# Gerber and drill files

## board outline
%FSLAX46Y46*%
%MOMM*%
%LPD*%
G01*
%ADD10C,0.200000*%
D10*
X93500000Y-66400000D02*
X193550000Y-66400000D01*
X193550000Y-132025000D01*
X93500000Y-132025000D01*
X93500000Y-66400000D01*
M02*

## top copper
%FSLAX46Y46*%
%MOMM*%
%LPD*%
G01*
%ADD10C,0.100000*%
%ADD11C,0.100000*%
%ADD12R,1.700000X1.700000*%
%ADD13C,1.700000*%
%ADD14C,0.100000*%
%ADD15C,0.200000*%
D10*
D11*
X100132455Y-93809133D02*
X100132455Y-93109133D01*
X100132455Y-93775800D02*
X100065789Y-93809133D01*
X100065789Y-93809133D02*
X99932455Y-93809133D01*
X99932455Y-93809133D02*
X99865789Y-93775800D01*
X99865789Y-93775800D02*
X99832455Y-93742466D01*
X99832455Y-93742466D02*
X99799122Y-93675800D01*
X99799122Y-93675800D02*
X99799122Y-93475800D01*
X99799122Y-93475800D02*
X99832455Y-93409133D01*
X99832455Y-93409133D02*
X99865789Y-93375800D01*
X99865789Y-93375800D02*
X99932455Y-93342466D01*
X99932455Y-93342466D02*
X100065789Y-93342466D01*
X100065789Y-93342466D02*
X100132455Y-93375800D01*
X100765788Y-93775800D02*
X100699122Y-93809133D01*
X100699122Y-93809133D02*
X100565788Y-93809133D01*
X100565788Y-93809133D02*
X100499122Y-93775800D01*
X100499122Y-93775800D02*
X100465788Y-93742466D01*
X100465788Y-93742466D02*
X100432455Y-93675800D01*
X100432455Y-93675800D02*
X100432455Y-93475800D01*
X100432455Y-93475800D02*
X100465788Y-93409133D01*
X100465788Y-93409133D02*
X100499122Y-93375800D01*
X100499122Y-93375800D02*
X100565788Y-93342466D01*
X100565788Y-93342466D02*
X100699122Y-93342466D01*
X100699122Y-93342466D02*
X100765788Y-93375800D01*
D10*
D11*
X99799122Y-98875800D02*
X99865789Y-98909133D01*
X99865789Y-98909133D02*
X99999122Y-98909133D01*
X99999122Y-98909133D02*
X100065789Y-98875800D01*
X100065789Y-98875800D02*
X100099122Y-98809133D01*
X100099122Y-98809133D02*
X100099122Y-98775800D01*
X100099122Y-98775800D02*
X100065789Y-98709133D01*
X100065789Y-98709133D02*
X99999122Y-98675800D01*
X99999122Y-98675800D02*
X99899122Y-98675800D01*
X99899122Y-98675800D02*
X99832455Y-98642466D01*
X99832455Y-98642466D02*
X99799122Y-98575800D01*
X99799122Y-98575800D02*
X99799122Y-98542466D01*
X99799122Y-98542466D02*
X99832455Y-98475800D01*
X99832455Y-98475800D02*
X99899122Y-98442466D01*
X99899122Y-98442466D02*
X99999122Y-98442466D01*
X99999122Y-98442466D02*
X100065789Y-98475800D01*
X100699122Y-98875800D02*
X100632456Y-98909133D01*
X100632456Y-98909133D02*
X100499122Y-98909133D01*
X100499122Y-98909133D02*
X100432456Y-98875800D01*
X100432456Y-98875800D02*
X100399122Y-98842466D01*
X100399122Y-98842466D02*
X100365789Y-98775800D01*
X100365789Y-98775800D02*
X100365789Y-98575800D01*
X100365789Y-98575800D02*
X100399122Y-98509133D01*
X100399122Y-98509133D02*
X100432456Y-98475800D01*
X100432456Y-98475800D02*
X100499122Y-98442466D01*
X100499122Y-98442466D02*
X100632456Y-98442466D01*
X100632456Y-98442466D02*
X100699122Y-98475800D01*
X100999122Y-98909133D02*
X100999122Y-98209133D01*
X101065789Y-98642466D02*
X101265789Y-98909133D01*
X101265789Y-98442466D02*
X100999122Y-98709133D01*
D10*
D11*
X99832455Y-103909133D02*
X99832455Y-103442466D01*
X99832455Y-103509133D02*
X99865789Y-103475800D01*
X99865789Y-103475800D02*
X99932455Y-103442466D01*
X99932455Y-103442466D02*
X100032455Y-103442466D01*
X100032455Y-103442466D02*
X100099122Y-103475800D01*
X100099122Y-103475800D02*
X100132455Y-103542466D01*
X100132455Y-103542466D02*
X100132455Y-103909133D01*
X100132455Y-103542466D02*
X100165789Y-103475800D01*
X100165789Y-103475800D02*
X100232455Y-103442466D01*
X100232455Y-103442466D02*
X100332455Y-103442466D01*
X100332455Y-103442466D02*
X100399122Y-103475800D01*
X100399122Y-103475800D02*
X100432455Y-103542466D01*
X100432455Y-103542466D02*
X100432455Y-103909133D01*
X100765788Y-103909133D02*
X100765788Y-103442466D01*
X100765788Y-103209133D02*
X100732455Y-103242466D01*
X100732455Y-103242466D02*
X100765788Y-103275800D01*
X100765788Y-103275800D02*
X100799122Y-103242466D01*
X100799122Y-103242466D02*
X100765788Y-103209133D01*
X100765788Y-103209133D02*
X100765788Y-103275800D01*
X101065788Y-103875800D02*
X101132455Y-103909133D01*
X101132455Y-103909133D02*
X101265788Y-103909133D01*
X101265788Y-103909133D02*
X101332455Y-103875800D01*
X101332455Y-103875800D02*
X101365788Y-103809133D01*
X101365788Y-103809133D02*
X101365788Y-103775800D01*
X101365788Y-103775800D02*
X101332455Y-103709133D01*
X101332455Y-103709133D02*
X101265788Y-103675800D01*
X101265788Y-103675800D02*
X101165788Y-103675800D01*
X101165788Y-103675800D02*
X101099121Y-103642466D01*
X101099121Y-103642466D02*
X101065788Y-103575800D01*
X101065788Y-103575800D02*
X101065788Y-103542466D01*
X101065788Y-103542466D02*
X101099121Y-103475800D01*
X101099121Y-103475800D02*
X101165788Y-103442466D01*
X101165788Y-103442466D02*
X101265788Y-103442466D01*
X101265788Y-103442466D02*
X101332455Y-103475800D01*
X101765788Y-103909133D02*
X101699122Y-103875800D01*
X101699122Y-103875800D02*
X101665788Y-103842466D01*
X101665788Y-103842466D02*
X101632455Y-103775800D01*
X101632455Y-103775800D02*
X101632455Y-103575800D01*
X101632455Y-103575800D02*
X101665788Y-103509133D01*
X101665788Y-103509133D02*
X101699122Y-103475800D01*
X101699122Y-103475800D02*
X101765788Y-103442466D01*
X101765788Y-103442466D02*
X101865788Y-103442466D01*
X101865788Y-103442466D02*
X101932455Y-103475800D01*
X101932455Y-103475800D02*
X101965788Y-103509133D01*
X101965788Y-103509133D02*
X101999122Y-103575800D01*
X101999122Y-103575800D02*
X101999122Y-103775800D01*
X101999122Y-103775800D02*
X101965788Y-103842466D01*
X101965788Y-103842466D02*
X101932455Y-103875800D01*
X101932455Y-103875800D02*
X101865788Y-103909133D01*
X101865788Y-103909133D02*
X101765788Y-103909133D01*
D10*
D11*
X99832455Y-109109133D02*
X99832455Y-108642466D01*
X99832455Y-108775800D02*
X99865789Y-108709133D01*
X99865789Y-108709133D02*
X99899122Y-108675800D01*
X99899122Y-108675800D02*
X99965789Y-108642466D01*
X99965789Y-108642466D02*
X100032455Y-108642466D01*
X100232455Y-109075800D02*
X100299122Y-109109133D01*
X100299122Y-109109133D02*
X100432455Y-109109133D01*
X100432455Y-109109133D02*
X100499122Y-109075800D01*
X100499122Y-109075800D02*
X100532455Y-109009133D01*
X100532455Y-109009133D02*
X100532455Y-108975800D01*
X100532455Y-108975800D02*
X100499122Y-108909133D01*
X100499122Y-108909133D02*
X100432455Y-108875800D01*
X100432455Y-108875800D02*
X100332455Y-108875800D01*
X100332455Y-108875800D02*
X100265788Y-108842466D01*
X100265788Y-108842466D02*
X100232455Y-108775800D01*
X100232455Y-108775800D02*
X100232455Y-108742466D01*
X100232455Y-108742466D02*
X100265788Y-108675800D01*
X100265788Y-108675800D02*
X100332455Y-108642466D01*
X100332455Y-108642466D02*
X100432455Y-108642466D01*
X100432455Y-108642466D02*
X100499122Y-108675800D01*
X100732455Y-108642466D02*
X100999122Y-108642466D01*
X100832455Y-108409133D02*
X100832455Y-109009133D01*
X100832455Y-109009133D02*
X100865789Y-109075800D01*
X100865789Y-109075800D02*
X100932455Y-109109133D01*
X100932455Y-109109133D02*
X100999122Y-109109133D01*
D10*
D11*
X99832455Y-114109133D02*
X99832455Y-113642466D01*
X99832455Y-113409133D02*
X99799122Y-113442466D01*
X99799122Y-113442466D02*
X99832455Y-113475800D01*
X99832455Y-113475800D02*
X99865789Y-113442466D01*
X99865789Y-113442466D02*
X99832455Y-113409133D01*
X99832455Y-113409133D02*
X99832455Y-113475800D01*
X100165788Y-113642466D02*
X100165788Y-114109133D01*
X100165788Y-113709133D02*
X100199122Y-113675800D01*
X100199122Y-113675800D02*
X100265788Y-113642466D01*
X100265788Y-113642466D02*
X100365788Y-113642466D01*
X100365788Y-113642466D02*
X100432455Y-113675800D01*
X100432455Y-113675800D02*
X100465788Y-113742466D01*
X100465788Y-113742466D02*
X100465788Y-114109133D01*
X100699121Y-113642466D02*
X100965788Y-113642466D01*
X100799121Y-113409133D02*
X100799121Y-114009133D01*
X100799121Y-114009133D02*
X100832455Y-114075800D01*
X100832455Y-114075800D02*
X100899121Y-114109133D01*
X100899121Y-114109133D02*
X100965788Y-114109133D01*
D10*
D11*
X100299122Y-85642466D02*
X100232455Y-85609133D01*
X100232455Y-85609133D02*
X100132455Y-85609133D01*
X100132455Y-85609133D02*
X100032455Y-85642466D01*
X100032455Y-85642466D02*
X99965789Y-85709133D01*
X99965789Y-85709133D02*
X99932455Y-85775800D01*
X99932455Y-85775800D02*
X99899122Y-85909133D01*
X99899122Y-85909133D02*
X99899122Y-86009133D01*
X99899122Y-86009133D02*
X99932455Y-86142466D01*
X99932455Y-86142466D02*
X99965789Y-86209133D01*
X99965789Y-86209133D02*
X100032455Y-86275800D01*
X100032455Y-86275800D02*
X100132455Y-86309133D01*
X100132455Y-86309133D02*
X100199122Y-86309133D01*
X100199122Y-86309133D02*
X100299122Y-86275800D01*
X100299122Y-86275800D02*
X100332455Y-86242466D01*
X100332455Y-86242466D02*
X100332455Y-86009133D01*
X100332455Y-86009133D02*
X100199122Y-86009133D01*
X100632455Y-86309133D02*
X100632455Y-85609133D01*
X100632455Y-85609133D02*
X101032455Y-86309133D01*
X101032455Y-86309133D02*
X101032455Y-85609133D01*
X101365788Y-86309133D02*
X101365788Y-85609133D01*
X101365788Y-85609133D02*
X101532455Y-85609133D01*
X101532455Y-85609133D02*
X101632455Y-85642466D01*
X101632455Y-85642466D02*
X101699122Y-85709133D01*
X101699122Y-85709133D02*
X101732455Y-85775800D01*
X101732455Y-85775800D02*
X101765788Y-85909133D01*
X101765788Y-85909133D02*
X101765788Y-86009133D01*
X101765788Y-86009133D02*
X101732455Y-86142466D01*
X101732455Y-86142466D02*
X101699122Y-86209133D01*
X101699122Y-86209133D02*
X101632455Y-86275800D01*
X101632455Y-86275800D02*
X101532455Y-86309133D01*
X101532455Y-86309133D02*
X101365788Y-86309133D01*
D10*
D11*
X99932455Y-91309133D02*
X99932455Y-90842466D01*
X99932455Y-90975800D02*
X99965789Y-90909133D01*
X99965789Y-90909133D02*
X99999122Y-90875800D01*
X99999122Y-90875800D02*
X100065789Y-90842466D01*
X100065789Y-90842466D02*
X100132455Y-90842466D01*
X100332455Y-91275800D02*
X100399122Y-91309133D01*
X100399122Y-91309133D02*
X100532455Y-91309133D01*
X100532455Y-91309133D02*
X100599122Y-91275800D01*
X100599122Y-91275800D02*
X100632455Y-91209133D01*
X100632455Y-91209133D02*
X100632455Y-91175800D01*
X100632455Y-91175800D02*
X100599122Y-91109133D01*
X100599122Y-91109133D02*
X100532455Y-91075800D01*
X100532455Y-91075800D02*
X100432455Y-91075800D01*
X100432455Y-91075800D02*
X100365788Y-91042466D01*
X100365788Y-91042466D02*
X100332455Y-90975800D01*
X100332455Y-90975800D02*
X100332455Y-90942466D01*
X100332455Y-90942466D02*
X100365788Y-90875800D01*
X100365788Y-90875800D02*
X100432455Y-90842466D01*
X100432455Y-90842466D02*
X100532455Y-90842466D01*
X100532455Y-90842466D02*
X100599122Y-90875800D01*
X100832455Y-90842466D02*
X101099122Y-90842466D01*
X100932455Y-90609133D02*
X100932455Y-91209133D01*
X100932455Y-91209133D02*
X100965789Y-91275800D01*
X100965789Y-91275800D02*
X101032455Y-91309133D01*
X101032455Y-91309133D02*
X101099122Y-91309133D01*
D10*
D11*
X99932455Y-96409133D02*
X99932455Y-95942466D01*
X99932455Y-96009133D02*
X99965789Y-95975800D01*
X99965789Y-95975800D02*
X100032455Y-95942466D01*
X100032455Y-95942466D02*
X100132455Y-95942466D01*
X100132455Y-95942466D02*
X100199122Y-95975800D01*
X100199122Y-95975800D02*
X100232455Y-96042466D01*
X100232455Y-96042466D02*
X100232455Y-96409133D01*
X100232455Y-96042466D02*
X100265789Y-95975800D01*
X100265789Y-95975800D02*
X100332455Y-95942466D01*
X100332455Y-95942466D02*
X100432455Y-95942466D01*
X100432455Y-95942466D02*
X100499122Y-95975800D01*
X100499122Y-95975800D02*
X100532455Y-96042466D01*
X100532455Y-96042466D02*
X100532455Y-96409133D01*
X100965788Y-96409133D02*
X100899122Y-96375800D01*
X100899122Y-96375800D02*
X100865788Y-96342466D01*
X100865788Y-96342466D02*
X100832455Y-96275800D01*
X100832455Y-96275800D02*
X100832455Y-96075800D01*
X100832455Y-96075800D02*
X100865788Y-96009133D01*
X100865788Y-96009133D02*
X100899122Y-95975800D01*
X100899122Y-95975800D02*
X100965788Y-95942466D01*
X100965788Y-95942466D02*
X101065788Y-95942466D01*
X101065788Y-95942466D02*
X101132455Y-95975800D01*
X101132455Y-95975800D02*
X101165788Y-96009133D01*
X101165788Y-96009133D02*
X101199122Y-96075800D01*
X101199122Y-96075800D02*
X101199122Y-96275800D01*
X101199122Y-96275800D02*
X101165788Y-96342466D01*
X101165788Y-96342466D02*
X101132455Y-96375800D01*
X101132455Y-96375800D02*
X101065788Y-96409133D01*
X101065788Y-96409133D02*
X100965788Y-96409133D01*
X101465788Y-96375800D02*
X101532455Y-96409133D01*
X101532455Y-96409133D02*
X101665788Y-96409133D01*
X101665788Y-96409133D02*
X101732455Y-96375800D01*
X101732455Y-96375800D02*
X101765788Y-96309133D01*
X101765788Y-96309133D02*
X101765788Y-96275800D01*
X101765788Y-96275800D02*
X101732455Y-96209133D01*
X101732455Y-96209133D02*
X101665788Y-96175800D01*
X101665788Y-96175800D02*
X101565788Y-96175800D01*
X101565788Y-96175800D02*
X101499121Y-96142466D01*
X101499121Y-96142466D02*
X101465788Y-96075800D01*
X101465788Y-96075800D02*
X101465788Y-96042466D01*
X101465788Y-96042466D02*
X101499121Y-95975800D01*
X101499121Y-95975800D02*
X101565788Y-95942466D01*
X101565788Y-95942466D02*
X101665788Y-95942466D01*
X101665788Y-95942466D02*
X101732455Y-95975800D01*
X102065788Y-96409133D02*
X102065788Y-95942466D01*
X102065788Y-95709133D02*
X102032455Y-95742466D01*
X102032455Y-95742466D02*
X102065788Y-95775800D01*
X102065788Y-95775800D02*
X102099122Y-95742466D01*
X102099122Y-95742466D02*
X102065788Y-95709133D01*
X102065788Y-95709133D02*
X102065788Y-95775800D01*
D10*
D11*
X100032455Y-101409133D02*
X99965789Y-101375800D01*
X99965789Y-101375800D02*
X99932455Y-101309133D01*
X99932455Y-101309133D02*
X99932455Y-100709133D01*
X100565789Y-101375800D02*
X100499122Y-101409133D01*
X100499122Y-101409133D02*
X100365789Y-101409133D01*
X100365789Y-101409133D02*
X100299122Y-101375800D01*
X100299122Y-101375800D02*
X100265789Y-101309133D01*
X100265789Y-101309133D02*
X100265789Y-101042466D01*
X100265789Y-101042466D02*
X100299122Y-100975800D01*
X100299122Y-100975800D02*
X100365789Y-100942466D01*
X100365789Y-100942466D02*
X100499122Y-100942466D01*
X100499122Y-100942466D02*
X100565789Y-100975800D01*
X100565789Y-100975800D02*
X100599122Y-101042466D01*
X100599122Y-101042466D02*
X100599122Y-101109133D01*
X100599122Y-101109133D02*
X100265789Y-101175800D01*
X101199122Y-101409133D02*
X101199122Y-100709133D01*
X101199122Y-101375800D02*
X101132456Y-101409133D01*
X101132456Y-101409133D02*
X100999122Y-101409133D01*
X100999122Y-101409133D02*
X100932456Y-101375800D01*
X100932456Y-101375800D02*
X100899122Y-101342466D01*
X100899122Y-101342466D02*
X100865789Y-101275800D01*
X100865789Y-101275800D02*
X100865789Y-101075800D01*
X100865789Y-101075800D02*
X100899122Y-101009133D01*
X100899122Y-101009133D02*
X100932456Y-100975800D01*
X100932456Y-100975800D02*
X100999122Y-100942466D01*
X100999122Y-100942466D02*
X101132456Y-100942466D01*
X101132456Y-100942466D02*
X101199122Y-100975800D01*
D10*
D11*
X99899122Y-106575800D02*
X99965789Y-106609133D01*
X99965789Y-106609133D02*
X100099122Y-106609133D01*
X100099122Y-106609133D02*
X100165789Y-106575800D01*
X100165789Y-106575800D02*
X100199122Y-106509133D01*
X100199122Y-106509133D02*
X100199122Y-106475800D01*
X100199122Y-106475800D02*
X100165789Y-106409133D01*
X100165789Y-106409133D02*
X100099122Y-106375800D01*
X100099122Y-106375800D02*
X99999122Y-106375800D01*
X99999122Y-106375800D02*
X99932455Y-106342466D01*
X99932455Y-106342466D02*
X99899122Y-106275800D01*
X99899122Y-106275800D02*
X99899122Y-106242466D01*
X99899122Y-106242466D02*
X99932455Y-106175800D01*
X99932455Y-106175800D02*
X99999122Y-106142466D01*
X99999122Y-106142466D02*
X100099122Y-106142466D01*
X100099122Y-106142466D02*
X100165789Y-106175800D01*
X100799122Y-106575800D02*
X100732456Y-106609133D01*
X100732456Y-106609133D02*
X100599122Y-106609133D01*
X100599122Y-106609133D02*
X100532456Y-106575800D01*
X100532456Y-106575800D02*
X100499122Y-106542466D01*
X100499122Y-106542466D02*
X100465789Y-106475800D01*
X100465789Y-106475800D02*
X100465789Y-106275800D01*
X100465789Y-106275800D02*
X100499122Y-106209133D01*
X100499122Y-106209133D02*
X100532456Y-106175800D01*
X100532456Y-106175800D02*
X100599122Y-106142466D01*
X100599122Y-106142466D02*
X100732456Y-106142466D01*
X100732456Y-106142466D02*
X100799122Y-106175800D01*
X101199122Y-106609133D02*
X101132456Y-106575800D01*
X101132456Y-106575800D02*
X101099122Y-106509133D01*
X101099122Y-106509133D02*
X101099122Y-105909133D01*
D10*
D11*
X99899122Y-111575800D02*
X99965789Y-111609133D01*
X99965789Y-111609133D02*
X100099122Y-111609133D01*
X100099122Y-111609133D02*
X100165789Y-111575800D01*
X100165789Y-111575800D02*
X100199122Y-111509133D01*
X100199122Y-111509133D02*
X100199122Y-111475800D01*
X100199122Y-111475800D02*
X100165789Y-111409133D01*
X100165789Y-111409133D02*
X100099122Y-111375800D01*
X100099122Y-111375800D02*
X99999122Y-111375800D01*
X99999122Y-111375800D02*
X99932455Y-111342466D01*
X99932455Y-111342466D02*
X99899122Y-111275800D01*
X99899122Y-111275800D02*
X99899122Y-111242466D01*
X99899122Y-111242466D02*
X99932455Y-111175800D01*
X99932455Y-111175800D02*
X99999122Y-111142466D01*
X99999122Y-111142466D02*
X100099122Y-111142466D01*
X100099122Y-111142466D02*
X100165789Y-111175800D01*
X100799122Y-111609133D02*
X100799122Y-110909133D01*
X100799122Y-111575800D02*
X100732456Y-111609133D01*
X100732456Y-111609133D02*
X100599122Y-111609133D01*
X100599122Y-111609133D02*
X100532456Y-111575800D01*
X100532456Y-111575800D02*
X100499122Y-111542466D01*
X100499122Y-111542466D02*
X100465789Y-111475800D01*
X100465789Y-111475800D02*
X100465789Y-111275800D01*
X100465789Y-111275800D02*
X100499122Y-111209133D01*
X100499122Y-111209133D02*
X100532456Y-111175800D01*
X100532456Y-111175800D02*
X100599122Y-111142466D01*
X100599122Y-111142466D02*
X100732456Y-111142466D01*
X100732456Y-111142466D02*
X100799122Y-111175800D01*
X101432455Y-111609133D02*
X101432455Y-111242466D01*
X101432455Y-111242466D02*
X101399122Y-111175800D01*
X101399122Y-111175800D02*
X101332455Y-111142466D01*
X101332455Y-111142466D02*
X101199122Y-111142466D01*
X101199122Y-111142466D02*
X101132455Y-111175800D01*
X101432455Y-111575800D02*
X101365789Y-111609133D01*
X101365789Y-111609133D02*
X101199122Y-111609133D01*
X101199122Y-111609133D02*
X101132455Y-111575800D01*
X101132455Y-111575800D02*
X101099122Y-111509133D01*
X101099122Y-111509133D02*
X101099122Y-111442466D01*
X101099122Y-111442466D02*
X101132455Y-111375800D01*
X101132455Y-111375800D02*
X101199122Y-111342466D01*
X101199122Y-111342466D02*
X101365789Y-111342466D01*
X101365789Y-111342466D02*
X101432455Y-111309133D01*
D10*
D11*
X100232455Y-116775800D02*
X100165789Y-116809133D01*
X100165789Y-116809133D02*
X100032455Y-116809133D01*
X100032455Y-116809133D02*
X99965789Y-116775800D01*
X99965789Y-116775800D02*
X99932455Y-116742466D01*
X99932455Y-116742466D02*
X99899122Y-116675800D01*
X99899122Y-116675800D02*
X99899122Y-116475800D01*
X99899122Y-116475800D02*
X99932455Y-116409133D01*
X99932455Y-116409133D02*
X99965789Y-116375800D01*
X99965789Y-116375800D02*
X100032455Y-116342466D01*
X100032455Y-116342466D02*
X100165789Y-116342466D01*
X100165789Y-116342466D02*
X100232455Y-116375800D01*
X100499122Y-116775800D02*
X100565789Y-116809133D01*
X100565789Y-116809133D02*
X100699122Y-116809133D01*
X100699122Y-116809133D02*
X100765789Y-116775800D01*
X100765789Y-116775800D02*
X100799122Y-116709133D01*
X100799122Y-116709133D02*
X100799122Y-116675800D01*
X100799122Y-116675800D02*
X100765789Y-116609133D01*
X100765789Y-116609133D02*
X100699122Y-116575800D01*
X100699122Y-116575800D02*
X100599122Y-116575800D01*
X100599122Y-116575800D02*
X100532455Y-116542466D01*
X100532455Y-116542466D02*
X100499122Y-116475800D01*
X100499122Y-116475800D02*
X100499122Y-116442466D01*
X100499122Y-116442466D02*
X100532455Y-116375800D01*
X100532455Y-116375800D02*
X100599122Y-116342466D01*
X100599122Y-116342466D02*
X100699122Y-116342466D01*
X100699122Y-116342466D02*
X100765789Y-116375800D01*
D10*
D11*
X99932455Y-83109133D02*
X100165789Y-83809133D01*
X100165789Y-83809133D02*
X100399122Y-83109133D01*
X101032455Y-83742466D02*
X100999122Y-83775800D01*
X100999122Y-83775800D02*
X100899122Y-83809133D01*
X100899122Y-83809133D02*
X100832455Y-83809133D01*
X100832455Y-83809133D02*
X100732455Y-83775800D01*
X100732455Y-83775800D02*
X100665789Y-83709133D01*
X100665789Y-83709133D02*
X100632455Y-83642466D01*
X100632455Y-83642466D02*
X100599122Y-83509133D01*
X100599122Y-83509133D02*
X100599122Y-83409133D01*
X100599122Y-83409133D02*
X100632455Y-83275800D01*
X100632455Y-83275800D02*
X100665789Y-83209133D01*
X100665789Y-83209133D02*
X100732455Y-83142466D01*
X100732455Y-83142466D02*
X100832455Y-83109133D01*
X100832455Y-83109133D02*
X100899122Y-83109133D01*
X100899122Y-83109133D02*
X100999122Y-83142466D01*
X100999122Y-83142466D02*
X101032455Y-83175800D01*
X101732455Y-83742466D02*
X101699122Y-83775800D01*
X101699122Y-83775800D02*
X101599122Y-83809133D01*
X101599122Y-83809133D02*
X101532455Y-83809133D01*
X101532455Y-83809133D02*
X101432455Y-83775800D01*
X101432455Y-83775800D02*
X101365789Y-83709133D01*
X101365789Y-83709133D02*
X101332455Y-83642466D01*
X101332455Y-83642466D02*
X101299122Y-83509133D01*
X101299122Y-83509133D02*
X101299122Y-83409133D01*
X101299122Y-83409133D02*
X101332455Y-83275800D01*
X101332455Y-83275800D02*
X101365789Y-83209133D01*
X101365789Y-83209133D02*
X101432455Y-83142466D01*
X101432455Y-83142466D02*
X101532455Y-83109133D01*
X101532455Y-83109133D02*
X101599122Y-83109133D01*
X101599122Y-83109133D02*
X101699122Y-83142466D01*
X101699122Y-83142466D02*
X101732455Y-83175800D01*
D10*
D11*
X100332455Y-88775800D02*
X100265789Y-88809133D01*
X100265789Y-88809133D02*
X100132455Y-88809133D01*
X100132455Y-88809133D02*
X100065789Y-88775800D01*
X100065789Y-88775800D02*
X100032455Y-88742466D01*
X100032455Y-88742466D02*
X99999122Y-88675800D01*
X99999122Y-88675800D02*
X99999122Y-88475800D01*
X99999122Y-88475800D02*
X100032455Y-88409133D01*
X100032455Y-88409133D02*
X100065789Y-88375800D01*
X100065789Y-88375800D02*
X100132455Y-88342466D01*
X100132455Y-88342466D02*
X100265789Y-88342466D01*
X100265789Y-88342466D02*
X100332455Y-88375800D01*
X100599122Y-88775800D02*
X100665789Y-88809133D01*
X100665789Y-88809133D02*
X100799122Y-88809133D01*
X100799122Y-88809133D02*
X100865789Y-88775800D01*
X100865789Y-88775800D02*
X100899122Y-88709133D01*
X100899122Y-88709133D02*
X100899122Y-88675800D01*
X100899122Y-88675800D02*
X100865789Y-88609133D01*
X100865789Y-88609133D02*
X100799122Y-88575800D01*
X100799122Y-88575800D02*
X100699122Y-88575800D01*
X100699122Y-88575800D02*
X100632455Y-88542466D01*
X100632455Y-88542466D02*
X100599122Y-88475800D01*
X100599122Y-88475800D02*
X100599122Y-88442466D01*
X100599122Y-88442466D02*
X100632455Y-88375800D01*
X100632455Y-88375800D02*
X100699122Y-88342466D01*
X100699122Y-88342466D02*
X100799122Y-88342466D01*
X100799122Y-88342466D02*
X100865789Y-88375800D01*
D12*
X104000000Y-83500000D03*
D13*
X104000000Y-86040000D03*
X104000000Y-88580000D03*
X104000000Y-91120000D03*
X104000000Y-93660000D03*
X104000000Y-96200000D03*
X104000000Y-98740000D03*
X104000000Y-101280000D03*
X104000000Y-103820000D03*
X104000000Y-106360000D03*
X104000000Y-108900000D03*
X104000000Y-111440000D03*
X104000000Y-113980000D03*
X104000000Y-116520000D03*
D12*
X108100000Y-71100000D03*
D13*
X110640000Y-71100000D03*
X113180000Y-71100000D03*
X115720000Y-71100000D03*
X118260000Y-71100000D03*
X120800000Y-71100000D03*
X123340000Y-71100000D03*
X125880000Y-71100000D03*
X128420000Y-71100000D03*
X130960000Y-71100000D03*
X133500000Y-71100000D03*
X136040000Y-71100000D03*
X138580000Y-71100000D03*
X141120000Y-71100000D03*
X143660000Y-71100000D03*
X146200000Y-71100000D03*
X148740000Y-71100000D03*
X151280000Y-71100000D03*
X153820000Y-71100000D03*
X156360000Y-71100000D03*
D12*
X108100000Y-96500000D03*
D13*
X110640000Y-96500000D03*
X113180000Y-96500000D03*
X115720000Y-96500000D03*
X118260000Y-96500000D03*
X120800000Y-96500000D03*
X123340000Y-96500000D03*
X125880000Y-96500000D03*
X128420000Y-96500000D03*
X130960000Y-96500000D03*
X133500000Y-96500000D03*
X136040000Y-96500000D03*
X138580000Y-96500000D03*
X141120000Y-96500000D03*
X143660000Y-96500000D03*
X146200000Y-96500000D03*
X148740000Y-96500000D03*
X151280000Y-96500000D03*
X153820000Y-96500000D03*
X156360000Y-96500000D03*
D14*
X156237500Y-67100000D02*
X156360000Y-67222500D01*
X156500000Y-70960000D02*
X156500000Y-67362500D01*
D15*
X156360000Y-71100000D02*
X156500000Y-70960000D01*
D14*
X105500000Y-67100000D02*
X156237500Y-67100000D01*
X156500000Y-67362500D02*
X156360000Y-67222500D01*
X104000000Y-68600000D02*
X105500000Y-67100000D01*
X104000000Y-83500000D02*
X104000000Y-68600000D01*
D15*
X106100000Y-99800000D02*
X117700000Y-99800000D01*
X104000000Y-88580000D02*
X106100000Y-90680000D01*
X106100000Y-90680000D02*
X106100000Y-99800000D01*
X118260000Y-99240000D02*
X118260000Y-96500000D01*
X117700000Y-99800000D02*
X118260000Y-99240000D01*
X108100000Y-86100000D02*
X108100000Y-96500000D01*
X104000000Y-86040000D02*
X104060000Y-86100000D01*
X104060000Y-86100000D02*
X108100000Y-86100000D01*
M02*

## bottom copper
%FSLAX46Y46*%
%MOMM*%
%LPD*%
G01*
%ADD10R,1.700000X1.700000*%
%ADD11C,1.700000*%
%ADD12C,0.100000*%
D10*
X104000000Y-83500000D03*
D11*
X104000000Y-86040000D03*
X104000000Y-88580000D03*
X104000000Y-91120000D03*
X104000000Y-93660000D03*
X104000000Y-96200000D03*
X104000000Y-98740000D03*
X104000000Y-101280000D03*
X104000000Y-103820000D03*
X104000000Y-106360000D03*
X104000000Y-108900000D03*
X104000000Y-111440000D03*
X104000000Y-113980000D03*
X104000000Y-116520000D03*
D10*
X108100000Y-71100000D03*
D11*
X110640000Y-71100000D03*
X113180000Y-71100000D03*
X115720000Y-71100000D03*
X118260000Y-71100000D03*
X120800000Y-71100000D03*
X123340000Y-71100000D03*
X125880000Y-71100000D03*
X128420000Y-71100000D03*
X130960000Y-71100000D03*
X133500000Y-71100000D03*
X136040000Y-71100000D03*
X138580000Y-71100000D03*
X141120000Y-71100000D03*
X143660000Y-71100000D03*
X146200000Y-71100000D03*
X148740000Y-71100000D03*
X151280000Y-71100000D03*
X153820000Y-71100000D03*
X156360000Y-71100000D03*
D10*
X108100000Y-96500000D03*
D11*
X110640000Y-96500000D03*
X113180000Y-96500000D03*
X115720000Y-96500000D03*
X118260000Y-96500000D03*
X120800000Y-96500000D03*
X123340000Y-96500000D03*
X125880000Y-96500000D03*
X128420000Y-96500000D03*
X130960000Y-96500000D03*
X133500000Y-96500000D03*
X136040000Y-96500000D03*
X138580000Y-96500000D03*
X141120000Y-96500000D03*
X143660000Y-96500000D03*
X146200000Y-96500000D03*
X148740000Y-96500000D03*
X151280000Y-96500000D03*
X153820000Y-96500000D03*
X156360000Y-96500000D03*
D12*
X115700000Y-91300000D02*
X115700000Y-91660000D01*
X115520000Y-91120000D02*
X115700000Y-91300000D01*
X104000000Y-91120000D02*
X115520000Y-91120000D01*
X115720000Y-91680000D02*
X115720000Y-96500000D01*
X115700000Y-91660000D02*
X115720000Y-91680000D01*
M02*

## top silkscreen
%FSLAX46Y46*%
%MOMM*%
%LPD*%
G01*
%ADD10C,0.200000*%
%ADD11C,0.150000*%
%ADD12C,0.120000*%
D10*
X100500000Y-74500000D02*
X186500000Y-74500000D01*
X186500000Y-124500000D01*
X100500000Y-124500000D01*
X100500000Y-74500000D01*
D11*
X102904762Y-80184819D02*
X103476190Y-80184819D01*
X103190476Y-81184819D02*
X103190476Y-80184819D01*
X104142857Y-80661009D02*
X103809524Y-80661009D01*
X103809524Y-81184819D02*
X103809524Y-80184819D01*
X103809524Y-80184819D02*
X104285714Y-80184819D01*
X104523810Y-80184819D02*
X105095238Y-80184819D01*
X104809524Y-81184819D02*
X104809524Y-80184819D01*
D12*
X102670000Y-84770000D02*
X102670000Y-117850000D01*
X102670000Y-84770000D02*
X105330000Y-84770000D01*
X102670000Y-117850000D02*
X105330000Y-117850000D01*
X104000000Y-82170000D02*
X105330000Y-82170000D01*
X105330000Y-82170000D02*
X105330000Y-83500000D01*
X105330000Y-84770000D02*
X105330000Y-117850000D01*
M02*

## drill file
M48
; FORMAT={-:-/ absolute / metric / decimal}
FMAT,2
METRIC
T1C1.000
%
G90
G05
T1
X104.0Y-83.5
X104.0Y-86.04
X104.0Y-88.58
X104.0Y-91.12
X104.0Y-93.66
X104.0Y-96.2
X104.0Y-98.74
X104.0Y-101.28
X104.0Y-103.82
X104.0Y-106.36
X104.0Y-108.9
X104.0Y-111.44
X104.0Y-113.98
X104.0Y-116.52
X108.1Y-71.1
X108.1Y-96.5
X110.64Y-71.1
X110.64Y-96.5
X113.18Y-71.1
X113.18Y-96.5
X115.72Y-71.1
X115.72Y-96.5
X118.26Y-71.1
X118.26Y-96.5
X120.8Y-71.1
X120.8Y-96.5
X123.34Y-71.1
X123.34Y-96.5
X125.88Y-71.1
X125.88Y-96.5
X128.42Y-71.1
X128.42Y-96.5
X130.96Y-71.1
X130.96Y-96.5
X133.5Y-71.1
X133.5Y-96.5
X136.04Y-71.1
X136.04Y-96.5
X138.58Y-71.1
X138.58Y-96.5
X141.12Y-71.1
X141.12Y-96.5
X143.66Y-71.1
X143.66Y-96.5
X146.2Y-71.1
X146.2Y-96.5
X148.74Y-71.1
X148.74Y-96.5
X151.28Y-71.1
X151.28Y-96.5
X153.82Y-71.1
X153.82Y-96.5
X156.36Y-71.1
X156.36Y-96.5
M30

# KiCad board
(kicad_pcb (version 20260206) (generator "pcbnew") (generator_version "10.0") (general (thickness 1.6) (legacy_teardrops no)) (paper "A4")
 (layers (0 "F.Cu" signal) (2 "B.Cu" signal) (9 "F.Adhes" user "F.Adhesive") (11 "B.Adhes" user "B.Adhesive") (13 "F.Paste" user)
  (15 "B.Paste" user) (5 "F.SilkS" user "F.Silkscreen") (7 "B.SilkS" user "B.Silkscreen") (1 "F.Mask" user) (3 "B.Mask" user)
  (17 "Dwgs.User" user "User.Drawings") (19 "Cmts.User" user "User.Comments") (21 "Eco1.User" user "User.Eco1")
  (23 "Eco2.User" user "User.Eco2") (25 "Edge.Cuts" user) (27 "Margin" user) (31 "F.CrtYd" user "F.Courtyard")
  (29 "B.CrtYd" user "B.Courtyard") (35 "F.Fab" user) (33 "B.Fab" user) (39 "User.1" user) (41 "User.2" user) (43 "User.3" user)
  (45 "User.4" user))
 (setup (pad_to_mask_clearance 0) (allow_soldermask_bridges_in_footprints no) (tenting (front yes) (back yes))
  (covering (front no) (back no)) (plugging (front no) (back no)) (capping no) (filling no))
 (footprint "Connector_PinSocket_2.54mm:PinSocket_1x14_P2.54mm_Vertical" (layer "F.Cu") (at 104 83.5)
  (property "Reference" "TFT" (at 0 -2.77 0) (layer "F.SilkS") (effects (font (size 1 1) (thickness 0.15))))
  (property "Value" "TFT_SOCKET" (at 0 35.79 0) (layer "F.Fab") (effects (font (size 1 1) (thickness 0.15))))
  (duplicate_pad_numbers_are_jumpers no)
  (fp_line (start -1.33 1.27) (end -1.33 34.35) (stroke (width 0.12) (type solid)) (layer "F.SilkS"))
  (fp_line (start -1.33 1.27) (end 1.33 1.27) (stroke (width 0.12) (type solid)) (layer "F.SilkS"))
  (fp_line (start -1.33 34.35) (end 1.33 34.35) (stroke (width 0.12) (type solid)) (layer "F.SilkS"))
  (fp_line (start 0 -1.33) (end 1.33 -1.33) (stroke (width 0.12) (type solid)) (layer "F.SilkS"))
  (fp_line (start 1.33 -1.33) (end 1.33 0) (stroke (width 0.12) (type solid)) (layer "F.SilkS"))
  (fp_line (start 1.33 1.27) (end 1.33 34.35) (stroke (width 0.12) (type solid)) (layer "F.SilkS"))
  (pad "1" thru_hole rect (at 0 0) (size 1.7 1.7) (drill 1) (layers "*.Cu" "*.Mask") (remove_unused_layers no) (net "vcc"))
  (pad "2" thru_hole circle (at 0 2.54) (size 1.7 1.7) (drill 1) (layers "*.Cu" "*.Mask") (remove_unused_layers no) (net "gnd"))
  (pad "3" thru_hole circle (at 0 5.08) (size 1.7 1.7) (drill 1) (layers "*.Cu" "*.Mask") (remove_unused_layers no) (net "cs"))
  (pad "4" thru_hole circle (at 0 7.62) (size 1.7 1.7) (drill 1) (layers "*.Cu" "*.Mask") (remove_unused_layers no) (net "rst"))
  (pad "5" thru_hole circle (at 0 10.16) (size 1.7 1.7) (drill 1) (layers "*.Cu" "*.Mask") (remove_unused_layers no))
  (pad "6" thru_hole circle (at 0 12.7) (size 1.7 1.7) (drill 1) (layers "*.Cu" "*.Mask") (remove_unused_layers no))
  (pad "7" thru_hole circle (at 0 15.24) (size 1.7 1.7) (drill 1) (layers "*.Cu" "*.Mask") (remove_unused_layers no))
  (pad "8" thru_hole circle (at 0 17.78) (size 1.7 1.7) (drill 1) (layers "*.Cu" "*.Mask") (remove_unused_layers no))
  (pad "9" thru_hole circle (at 0 20.32) (size 1.7 1.7) (drill 1) (layers "*.Cu" "*.Mask") (remove_unused_layers no))
  (pad "10" thru_hole circle (at 0 22.86) (size 1.7 1.7) (drill 1) (layers "*.Cu" "*.Mask") (remove_unused_layers no))
  (pad "11" thru_hole circle (at 0 25.4) (size 1.7 1.7) (drill 1) (layers "*.Cu" "*.Mask") (remove_unused_layers no))
  (pad "12" thru_hole circle (at 0 27.94) (size 1.7 1.7) (drill 1) (layers "*.Cu" "*.Mask") (remove_unused_layers no))
  (pad "13" thru_hole circle (at 0 30.48) (size 1.7 1.7) (drill 1) (layers "*.Cu" "*.Mask") (remove_unused_layers no))
  (pad "14" thru_hole circle (at 0 33.02) (size 1.7 1.7) (drill 1) (layers "*.Cu" "*.Mask") (remove_unused_layers no)))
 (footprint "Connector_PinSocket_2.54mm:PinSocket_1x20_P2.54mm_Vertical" (layer "B.Cu") (at 108.1 71.1 -90)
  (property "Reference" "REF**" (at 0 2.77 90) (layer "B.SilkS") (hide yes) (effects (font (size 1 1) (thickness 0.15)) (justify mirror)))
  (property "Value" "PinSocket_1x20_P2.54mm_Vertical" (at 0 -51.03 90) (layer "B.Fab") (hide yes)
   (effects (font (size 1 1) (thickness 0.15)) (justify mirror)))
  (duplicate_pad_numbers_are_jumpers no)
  (pad "1" thru_hole rect (at 0 0 270) (size 1.7 1.7) (drill 1) (layers "*.Cu" "*.Mask") (remove_unused_layers no))
  (pad "2" thru_hole circle (at 0 -2.54 270) (size 1.7 1.7) (drill 1) (layers "*.Cu" "*.Mask") (remove_unused_layers no))
  (pad "3" thru_hole circle (at 0 -5.08 270) (size 1.7 1.7) (drill 1) (layers "*.Cu" "*.Mask") (remove_unused_layers no))
  (pad "4" thru_hole circle (at 0 -7.62 270) (size 1.7 1.7) (drill 1) (layers "*.Cu" "*.Mask") (remove_unused_layers no))
  (pad "5" thru_hole circle (at 0 -10.16 270) (size 1.7 1.7) (drill 1) (layers "*.Cu" "*.Mask") (remove_unused_layers no))
  (pad "6" thru_hole circle (at 0 -12.7 270) (size 1.7 1.7) (drill 1) (layers "*.Cu" "*.Mask") (remove_unused_layers no))
  (pad "7" thru_hole circle (at 0 -15.24 270) (size 1.7 1.7) (drill 1) (layers "*.Cu" "*.Mask") (remove_unused_layers no))
  (pad "8" thru_hole circle (at 0 -17.78 270) (size 1.7 1.7) (drill 1) (layers "*.Cu" "*.Mask") (remove_unused_layers no))
  (pad "9" thru_hole circle (at 0 -20.32 270) (size 1.7 1.7) (drill 1) (layers "*.Cu" "*.Mask") (remove_unused_layers no))
  (pad "10" thru_hole circle (at 0 -22.86 270) (size 1.7 1.7) (drill 1) (layers "*.Cu" "*.Mask") (remove_unused_layers no))
  (pad "11" thru_hole circle (at 0 -25.4 270) (size 1.7 1.7) (drill 1) (layers "*.Cu" "*.Mask") (remove_unused_layers no))
  (pad "12" thru_hole circle (at 0 -27.94 270) (size 1.7 1.7) (drill 1) (layers "*.Cu" "*.Mask") (remove_unused_layers no))
  (pad "13" thru_hole circle (at 0 -30.48 270) (size 1.7 1.7) (drill 1) (layers "*.Cu" "*.Mask") (remove_unused_layers no))
  (pad "14" thru_hole circle (at 0 -33.02 270) (size 1.7 1.7) (drill 1) (layers "*.Cu" "*.Mask") (remove_unused_layers no))
  (pad "15" thru_hole circle (at 0 -35.56 270) (size 1.7 1.7) (drill 1) (layers "*.Cu" "*.Mask") (remove_unused_layers no))
  (pad "16" thru_hole circle (at 0 -38.1 270) (size 1.7 1.7) (drill 1) (layers "*.Cu" "*.Mask") (remove_unused_layers no))
  (pad "17" thru_hole circle (at 0 -40.64 270) (size 1.7 1.7) (drill 1) (layers "*.Cu" "*.Mask") (remove_unused_layers no))
  (pad "18" thru_hole circle (at 0 -43.18 270) (size 1.7 1.7) (drill 1) (layers "*.Cu" "*.Mask") (remove_unused_layers no))
  (pad "19" thru_hole circle (at 0 -45.72 270) (size 1.7 1.7) (drill 1) (layers "*.Cu" "*.Mask") (remove_unused_layers no))
  (pad "20" thru_hole circle (at 0 -48.26 270) (size 1.7 1.7) (drill 1) (layers "*.Cu" "*.Mask") (remove_unused_layers no) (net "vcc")))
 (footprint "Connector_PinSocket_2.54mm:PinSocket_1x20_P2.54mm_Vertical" (layer "B.Cu") (at 108.1 96.5 -90)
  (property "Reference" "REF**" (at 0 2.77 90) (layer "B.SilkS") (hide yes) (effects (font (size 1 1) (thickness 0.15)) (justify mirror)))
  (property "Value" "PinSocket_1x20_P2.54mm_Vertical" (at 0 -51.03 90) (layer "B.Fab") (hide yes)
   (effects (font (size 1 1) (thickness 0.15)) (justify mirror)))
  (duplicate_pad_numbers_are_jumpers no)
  (pad "1" thru_hole rect (at 0 0 270) (size 1.7 1.7) (drill 1) (layers "*.Cu" "*.Mask") (remove_unused_layers no) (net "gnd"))
  (pad "2" thru_hole circle (at 0 -2.54 270) (size 1.7 1.7) (drill 1) (layers "*.Cu" "*.Mask") (remove_unused_layers no))
  (pad "3" thru_hole circle (at 0 -5.08 270) (size 1.7 1.7) (drill 1) (layers "*.Cu" "*.Mask") (remove_unused_layers no))
  (pad "4" thru_hole circle (at 0 -7.62 270) (size 1.7 1.7) (drill 1) (layers "*.Cu" "*.Mask") (remove_unused_layers no) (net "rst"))
  (pad "5" thru_hole circle (at 0 -10.16 270) (size 1.7 1.7) (drill 1) (layers "*.Cu" "*.Mask") (remove_unused_layers no) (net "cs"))
  (pad "6" thru_hole circle (at 0 -12.7 270) (size 1.7 1.7) (drill 1) (layers "*.Cu" "*.Mask") (remove_unused_layers no))
  (pad "7" thru_hole circle (at 0 -15.24 270) (size 1.7 1.7) (drill 1) (layers "*.Cu" "*.Mask") (remove_unused_layers no))
  (pad "8" thru_hole circle (at 0 -17.78 270) (size 1.7 1.7) (drill 1) (layers "*.Cu" "*.Mask") (remove_unused_layers no))
  (pad "9" thru_hole circle (at 0 -20.32 270) (size 1.7 1.7) (drill 1) (layers "*.Cu" "*.Mask") (remove_unused_layers no))
  (pad "10" thru_hole circle (at 0 -22.86 270) (size 1.7 1.7) (drill 1) (layers "*.Cu" "*.Mask") (remove_unused_layers no))
  (pad "11" thru_hole circle (at 0 -25.4 270) (size 1.7 1.7) (drill 1) (layers "*.Cu" "*.Mask") (remove_unused_layers no))
  (pad "12" thru_hole circle (at 0 -27.94 270) (size 1.7 1.7) (drill 1) (layers "*.Cu" "*.Mask") (remove_unused_layers no))
  (pad "13" thru_hole circle (at 0 -30.48 270) (size 1.7 1.7) (drill 1) (layers "*.Cu" "*.Mask") (remove_unused_layers no))
  (pad "14" thru_hole circle (at 0 -33.02 270) (size 1.7 1.7) (drill 1) (layers "*.Cu" "*.Mask") (remove_unused_layers no))
  (pad "15" thru_hole circle (at 0 -35.56 270) (size 1.7 1.7) (drill 1) (layers "*.Cu" "*.Mask") (remove_unused_layers no))
  (pad "16" thru_hole circle (at 0 -38.1 270) (size 1.7 1.7) (drill 1) (layers "*.Cu" "*.Mask") (remove_unused_layers no))
  (pad "17" thru_hole circle (at 0 -40.64 270) (size 1.7 1.7) (drill 1) (layers "*.Cu" "*.Mask") (remove_unused_layers no))
  (pad "18" thru_hole circle (at 0 -43.18 270) (size 1.7 1.7) (drill 1) (layers "*.Cu" "*.Mask") (remove_unused_layers no))
  (pad "19" thru_hole circle (at 0 -45.72 270) (size 1.7 1.7) (drill 1) (layers "*.Cu" "*.Mask") (remove_unused_layers no))
  (pad "20" thru_hole circle (at 0 -48.26 270) (size 1.7 1.7) (drill 1) (layers "*.Cu" "*.Mask") (remove_unused_layers no)))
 (gr_rect (start 100.5 74.5) (end 186.5 124.5) (stroke (width 0.2) (type default)) (fill no) (layer "F.SilkS"))
 (gr_rect (start 93.5 66.4) (end 193.55 132.025) (stroke (width 0.2) (type default)) (fill no) (layer "Edge.Cuts"))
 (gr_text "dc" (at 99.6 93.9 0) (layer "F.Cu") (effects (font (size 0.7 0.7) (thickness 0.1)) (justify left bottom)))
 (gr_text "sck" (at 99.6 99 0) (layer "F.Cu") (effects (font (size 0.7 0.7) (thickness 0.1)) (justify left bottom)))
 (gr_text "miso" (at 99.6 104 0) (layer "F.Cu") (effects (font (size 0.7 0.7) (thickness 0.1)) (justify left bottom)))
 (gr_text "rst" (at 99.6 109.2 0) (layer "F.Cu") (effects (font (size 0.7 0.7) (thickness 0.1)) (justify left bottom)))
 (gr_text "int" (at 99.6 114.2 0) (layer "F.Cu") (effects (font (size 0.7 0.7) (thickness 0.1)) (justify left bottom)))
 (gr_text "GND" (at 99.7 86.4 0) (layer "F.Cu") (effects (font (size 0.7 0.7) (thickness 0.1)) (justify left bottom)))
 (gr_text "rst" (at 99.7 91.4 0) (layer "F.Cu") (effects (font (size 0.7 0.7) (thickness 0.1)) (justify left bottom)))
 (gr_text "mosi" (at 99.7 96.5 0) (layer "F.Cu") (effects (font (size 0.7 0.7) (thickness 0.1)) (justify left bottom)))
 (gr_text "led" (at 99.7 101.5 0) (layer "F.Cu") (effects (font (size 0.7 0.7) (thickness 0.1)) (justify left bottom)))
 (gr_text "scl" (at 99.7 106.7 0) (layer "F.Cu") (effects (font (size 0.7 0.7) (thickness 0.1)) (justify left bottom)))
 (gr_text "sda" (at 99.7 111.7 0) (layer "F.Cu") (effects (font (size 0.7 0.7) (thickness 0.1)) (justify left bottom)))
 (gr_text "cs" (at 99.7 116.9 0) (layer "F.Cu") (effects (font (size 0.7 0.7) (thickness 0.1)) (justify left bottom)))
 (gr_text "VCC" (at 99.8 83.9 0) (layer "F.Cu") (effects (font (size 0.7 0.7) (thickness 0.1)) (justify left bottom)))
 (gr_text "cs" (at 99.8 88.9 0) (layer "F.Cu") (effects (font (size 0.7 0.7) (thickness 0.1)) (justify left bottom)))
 (segment (start 156.2375 67.1) (end 156.36 67.2225) (width 0.1) (layer "F.Cu") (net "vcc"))
 (segment (start 156.5 70.96) (end 156.5 67.3625) (width 0.1) (layer "F.Cu") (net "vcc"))
 (segment (start 156.36 71.1) (end 156.5 70.96) (width 0.2) (layer "F.Cu") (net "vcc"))
 (segment (start 105.5 67.1) (end 156.2375 67.1) (width 0.1) (layer "F.Cu") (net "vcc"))
 (segment (start 156.5 67.3625) (end 156.36 67.2225) (width 0.1) (layer "F.Cu") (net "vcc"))
 (segment (start 104 68.6) (end 105.5 67.1) (width 0.1) (layer "F.Cu") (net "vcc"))
 (segment (start 104 83.5) (end 104 68.6) (width 0.1) (layer "F.Cu") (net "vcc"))
 (segment (start 115.7 91.3) (end 115.7 91.66) (width 0.1) (layer "B.Cu") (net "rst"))
 (segment (start 115.52 91.12) (end 115.7 91.3) (width 0.1) (layer "B.Cu") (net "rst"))
 (segment (start 104 91.12) (end 115.52 91.12) (width 0.1) (layer "B.Cu") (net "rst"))
 (segment (start 115.72 91.68) (end 115.72 96.5) (width 0.1) (layer "B.Cu") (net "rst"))
 (segment (start 115.7 91.66) (end 115.72 91.68) (width 0.1) (layer "B.Cu") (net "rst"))
 (segment (start 106.1 99.8) (end 117.7 99.8) (width 0.2) (layer "F.Cu") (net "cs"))
 (segment (start 104 88.58) (end 106.1 90.68) (width 0.2) (layer "F.Cu") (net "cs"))
 (segment (start 106.1 90.68) (end 106.1 99.8) (width 0.2) (layer "F.Cu") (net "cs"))
 (segment (start 118.26 99.24) (end 118.26 96.5) (width 0.2) (layer "F.Cu") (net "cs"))
 (segment (start 117.7 99.8) (end 118.26 99.24) (width 0.2) (layer "F.Cu") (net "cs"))
 (segment (start 108.1 86.1) (end 108.1 96.5) (width 0.2) (layer "F.Cu") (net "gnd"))
 (segment (start 104 86.04) (end 104.06 86.1) (width 0.2) (layer "F.Cu") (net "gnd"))
 (segment (start 104.06 86.1) (end 108.1 86.1) (width 0.2) (layer "F.Cu") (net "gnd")))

